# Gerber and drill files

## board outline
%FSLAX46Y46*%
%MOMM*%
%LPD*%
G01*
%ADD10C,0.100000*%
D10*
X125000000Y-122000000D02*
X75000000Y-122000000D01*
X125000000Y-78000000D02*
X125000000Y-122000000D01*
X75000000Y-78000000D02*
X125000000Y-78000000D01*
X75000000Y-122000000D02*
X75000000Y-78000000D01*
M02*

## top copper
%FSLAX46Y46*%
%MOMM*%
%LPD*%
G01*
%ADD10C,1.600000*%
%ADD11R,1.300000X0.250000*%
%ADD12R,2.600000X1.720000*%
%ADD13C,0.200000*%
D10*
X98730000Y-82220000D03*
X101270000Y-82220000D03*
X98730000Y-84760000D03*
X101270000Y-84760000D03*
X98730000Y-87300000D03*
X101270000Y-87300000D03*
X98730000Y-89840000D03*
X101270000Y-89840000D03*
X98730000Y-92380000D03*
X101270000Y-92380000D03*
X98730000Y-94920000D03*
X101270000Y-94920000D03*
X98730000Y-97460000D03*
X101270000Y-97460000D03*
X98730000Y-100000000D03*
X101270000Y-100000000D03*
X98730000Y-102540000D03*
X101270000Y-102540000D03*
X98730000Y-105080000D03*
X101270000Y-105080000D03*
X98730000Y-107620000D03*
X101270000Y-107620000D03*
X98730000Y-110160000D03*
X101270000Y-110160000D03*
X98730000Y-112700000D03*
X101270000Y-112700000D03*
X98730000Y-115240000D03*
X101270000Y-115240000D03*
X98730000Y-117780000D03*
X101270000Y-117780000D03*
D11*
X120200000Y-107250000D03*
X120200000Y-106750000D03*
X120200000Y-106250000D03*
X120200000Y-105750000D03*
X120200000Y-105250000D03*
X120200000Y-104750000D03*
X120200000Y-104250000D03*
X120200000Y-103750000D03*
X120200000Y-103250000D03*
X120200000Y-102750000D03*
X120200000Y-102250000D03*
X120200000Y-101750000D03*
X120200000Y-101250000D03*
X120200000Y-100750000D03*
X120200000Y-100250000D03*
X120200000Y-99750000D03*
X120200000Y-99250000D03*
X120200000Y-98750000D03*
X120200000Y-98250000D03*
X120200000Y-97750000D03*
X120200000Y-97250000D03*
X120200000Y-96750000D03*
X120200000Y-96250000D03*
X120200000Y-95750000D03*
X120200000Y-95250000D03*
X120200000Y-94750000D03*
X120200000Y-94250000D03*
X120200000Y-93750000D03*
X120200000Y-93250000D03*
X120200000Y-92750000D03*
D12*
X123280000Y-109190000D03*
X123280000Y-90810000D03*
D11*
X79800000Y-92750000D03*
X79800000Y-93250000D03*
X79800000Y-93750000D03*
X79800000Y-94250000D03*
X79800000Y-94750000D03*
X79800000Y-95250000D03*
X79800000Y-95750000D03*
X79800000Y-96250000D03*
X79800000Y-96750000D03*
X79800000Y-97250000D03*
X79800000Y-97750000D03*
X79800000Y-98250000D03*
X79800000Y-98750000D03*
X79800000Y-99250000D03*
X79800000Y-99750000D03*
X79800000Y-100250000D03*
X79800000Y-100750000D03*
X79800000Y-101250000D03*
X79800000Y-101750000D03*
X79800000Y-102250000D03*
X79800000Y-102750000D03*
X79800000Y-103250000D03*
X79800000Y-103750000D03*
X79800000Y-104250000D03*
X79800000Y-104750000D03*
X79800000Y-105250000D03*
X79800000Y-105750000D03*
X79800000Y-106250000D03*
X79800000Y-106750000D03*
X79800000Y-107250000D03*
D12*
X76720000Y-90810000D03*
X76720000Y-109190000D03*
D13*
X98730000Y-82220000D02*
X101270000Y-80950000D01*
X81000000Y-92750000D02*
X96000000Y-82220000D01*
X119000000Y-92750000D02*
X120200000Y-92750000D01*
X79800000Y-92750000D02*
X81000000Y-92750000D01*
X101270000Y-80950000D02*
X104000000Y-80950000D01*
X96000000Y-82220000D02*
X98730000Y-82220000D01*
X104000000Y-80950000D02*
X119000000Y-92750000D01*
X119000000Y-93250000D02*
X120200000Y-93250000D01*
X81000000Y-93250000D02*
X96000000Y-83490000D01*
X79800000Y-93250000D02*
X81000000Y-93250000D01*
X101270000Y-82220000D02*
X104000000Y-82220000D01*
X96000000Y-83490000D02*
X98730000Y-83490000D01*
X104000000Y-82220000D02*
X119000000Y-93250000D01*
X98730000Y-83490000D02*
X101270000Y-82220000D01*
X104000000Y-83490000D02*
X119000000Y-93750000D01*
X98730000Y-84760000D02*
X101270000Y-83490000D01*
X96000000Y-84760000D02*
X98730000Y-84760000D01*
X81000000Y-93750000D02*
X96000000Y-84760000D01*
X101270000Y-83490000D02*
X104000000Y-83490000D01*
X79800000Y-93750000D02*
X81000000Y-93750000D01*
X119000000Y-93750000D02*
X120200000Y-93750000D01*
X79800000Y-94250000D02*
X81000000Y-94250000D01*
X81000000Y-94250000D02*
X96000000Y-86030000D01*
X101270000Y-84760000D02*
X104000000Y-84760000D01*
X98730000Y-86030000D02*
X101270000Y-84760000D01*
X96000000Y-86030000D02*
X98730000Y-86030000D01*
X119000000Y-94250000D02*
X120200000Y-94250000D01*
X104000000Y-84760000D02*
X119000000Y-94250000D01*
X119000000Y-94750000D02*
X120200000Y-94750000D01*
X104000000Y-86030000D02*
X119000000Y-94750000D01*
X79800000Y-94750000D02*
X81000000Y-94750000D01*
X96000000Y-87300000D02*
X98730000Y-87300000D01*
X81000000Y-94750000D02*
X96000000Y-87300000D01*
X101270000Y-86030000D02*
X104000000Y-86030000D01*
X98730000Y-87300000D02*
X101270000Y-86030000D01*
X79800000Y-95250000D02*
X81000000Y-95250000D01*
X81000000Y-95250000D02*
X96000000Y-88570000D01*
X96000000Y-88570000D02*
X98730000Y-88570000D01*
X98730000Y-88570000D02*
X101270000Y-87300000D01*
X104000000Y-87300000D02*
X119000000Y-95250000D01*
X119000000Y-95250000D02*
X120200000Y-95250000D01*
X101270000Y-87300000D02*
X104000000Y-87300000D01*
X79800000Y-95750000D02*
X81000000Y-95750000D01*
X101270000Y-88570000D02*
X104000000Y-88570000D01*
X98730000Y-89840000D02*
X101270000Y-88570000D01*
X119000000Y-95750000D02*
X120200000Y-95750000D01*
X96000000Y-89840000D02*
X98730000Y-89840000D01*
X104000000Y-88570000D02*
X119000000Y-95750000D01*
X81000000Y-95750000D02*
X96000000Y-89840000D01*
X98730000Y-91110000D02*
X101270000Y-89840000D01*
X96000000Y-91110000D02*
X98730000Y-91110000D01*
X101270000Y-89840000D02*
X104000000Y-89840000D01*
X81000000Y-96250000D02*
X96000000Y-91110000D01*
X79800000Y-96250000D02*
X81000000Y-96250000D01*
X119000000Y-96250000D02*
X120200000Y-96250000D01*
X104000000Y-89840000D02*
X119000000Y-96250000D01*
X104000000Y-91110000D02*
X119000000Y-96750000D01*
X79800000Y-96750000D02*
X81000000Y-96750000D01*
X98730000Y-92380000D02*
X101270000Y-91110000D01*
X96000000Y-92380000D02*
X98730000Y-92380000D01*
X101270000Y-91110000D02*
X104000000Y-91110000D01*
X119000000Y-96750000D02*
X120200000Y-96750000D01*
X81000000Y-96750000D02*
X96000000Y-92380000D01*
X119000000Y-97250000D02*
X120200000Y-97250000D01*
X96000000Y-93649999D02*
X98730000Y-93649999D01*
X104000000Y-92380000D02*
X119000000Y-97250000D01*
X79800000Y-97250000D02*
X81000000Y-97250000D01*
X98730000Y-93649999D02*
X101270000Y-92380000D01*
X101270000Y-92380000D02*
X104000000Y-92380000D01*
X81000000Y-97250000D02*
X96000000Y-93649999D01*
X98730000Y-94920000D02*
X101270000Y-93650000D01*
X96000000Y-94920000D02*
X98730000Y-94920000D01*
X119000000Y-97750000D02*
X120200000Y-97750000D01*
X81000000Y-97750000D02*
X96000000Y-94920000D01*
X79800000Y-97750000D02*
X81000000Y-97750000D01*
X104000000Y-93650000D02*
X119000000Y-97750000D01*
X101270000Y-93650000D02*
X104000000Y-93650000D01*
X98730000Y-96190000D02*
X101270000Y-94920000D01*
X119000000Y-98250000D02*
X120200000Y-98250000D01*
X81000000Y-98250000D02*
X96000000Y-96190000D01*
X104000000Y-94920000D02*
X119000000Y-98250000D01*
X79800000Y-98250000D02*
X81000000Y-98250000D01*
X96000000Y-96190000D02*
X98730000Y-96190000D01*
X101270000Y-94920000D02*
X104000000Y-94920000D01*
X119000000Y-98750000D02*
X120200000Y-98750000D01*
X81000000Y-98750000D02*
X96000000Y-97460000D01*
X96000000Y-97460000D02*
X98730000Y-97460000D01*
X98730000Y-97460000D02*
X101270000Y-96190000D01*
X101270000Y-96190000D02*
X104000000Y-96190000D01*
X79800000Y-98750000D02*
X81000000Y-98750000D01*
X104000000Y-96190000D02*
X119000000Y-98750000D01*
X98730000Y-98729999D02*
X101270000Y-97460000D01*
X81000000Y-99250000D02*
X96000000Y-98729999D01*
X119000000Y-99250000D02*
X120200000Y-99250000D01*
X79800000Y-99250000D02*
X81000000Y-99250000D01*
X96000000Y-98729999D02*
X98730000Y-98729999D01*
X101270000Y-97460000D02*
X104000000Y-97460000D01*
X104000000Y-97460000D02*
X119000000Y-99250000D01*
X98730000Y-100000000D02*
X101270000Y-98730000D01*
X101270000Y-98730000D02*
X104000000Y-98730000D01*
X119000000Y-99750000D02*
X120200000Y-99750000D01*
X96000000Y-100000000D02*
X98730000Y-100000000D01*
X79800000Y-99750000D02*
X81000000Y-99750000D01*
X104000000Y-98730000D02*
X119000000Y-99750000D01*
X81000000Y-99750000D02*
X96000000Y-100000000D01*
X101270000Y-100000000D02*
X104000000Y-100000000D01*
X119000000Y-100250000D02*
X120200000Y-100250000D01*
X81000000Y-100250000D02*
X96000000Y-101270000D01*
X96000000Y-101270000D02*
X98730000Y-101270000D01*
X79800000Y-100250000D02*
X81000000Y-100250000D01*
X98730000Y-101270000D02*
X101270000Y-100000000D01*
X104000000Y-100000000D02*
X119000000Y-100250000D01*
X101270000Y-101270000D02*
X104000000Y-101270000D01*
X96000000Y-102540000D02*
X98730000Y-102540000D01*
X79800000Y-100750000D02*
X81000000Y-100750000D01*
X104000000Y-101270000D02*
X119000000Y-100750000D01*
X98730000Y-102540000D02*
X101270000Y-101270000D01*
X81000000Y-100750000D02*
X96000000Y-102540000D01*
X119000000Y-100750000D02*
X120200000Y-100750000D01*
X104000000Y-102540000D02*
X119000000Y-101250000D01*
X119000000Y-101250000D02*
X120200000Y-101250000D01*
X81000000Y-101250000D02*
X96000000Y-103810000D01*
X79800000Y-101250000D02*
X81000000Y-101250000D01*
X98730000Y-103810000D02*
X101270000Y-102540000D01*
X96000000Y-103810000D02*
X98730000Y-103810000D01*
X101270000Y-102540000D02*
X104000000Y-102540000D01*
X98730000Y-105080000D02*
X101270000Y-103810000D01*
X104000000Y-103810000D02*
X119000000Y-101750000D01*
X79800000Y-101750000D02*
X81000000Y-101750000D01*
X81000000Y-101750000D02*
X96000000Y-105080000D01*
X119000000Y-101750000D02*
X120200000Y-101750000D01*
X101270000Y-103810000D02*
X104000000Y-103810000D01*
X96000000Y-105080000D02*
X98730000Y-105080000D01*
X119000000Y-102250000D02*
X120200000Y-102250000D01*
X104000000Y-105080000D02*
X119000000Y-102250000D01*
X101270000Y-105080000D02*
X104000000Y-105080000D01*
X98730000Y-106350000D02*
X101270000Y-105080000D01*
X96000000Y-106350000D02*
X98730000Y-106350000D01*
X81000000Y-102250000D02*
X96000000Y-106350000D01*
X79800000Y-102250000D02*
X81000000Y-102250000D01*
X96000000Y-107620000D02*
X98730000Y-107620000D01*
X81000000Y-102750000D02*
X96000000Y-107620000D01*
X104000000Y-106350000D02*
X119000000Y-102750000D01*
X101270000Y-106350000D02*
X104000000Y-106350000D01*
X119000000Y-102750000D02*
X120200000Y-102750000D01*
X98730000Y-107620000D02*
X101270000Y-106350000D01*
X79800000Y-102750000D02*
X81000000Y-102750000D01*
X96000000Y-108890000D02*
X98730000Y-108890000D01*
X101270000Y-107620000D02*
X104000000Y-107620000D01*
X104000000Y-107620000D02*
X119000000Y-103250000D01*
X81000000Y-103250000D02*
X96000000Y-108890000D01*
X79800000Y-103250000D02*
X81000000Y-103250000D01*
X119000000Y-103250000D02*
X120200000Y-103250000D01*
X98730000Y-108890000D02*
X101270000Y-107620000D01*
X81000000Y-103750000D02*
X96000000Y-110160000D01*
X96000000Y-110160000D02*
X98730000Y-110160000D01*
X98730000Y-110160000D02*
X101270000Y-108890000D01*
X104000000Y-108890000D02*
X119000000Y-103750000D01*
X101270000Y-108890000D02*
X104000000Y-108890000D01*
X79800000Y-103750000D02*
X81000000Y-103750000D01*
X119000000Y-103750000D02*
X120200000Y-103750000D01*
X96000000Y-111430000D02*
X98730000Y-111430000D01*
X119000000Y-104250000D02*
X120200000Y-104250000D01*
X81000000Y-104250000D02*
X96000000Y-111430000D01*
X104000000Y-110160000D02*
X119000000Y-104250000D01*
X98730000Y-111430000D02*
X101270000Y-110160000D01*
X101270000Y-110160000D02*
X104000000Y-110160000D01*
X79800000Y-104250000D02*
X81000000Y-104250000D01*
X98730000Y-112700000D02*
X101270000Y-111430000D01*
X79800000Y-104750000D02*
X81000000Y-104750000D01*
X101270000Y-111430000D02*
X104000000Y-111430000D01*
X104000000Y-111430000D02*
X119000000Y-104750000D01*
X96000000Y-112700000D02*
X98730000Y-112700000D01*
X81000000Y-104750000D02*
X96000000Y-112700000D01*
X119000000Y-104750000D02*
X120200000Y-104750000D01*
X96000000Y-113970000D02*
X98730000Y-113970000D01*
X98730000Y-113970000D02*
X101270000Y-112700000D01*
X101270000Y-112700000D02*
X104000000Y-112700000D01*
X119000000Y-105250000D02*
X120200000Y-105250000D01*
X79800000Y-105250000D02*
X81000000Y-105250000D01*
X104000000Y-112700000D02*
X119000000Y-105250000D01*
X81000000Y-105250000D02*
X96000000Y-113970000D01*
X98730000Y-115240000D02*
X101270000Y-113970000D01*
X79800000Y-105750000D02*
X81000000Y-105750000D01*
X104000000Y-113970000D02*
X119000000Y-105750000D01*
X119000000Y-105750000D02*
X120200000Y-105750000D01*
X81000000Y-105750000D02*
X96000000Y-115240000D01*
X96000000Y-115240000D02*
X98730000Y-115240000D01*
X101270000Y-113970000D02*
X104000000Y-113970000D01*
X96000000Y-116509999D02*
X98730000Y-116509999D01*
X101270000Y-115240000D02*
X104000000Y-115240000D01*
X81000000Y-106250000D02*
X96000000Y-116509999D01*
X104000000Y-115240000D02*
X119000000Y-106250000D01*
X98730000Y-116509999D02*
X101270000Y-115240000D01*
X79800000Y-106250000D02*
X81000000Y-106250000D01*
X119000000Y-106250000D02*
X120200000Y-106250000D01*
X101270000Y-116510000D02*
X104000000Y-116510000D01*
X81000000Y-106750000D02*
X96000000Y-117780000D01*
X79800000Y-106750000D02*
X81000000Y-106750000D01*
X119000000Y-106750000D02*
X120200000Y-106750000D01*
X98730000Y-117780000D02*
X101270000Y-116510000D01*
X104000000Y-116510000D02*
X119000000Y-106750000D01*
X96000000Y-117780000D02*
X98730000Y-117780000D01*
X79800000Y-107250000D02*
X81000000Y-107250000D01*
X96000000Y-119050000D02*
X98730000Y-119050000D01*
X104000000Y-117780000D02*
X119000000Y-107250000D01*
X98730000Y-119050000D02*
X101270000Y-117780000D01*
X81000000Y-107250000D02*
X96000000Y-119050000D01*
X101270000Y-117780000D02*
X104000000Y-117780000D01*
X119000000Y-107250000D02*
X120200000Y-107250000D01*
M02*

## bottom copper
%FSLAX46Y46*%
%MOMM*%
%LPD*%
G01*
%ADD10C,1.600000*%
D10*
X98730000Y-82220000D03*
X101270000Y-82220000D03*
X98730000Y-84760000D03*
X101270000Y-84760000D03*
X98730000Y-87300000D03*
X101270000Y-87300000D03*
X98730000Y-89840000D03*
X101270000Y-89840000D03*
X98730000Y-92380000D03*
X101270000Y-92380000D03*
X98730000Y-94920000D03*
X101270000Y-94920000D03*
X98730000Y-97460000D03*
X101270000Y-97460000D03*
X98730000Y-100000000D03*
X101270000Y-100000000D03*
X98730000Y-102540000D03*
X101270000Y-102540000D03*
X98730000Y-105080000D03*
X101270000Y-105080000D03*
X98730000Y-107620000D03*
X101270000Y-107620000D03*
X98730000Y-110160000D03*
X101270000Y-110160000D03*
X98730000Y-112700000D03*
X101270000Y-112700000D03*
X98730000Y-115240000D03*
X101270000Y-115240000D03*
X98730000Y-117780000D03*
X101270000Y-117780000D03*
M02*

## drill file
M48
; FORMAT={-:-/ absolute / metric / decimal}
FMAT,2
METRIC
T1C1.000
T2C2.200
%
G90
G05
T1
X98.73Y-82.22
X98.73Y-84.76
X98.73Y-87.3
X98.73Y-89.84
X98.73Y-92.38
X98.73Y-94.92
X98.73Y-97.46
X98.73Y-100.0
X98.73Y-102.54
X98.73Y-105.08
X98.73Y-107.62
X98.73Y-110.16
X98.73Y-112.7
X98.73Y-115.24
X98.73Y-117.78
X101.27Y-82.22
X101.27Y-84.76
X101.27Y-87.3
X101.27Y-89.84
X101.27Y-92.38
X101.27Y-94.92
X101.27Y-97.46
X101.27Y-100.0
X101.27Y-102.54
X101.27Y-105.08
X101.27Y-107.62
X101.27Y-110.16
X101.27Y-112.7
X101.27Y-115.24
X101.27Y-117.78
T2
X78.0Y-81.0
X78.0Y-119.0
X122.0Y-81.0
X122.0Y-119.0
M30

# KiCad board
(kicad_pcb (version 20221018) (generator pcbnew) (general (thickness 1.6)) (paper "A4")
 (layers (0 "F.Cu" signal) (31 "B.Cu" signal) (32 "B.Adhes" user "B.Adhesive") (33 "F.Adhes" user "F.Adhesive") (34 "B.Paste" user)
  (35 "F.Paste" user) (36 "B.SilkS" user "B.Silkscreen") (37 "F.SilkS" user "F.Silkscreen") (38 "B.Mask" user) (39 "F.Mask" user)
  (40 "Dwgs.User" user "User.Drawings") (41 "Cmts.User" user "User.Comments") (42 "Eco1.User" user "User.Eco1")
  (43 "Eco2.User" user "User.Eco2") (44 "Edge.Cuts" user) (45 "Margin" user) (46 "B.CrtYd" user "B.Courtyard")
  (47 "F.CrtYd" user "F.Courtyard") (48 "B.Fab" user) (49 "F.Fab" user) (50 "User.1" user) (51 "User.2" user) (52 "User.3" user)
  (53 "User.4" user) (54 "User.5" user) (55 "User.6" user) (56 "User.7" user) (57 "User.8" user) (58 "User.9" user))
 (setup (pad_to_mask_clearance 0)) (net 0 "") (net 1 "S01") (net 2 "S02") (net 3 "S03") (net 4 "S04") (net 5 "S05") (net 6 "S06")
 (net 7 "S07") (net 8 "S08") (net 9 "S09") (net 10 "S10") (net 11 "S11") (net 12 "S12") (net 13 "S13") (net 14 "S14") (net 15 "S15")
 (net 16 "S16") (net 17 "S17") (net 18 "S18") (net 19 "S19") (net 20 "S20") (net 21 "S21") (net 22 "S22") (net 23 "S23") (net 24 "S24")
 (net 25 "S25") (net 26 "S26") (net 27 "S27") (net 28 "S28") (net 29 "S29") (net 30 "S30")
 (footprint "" (layer "F.Cu") (at 122 119)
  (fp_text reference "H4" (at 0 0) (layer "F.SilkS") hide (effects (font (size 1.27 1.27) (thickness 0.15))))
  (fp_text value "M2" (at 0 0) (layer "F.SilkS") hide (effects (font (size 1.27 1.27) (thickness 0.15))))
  (pad "" np_thru_hole circle (at 0 0) (size 2.2 2.2) (drill 2.2) (layers "F&B.Cu" "*.Mask")))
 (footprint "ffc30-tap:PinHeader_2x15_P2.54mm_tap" (layer "F.Cu") (at 100 100)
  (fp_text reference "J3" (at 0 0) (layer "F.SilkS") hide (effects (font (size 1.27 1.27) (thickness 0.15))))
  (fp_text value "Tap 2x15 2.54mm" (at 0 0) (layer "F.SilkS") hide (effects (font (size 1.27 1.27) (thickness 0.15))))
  (pad "1" thru_hole circle (at -1.27 -17.78) (size 1.6 1.6) (drill 1) (layers "*.Cu" "*.Mask") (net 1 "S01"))
  (pad "2" thru_hole circle (at 1.27 -17.78) (size 1.6 1.6) (drill 1) (layers "*.Cu" "*.Mask") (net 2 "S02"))
  (pad "3" thru_hole circle (at -1.27 -15.24) (size 1.6 1.6) (drill 1) (layers "*.Cu" "*.Mask") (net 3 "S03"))
  (pad "4" thru_hole circle (at 1.27 -15.24) (size 1.6 1.6) (drill 1) (layers "*.Cu" "*.Mask") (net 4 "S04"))
  (pad "5" thru_hole circle (at -1.27 -12.7) (size 1.6 1.6) (drill 1) (layers "*.Cu" "*.Mask") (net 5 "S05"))
  (pad "6" thru_hole circle (at 1.27 -12.7) (size 1.6 1.6) (drill 1) (layers "*.Cu" "*.Mask") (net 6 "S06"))
  (pad "7" thru_hole circle (at -1.27 -10.16) (size 1.6 1.6) (drill 1) (layers "*.Cu" "*.Mask") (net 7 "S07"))
  (pad "8" thru_hole circle (at 1.27 -10.16) (size 1.6 1.6) (drill 1) (layers "*.Cu" "*.Mask") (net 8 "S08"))
  (pad "9" thru_hole circle (at -1.27 -7.62) (size 1.6 1.6) (drill 1) (layers "*.Cu" "*.Mask") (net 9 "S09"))
  (pad "10" thru_hole circle (at 1.27 -7.62) (size 1.6 1.6) (drill 1) (layers "*.Cu" "*.Mask") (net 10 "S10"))
  (pad "11" thru_hole circle (at -1.27 -5.08) (size 1.6 1.6) (drill 1) (layers "*.Cu" "*.Mask") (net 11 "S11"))
  (pad "12" thru_hole circle (at 1.27 -5.08) (size 1.6 1.6) (drill 1) (layers "*.Cu" "*.Mask") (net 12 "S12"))
  (pad "13" thru_hole circle (at -1.27 -2.54) (size 1.6 1.6) (drill 1) (layers "*.Cu" "*.Mask") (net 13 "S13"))
  (pad "14" thru_hole circle (at 1.27 -2.54) (size 1.6 1.6) (drill 1) (layers "*.Cu" "*.Mask") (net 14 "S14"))
  (pad "15" thru_hole circle (at -1.27 0) (size 1.6 1.6) (drill 1) (layers "*.Cu" "*.Mask") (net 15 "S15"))
  (pad "16" thru_hole circle (at 1.27 0) (size 1.6 1.6) (drill 1) (layers "*.Cu" "*.Mask") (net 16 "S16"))
  (pad "17" thru_hole circle (at -1.27 2.54) (size 1.6 1.6) (drill 1) (layers "*.Cu" "*.Mask") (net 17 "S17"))
  (pad "18" thru_hole circle (at 1.27 2.54) (size 1.6 1.6) (drill 1) (layers "*.Cu" "*.Mask") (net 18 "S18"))
  (pad "19" thru_hole circle (at -1.27 5.08) (size 1.6 1.6) (drill 1) (layers "*.Cu" "*.Mask") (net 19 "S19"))
  (pad "20" thru_hole circle (at 1.27 5.08) (size 1.6 1.6) (drill 1) (layers "*.Cu" "*.Mask") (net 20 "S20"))
  (pad "21" thru_hole circle (at -1.27 7.62) (size 1.6 1.6) (drill 1) (layers "*.Cu" "*.Mask") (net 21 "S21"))
  (pad "22" thru_hole circle (at 1.27 7.62) (size 1.6 1.6) (drill 1) (layers "*.Cu" "*.Mask") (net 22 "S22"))
  (pad "23" thru_hole circle (at -1.27 10.16) (size 1.6 1.6) (drill 1) (layers "*.Cu" "*.Mask") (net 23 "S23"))
  (pad "24" thru_hole circle (at 1.27 10.16) (size 1.6 1.6) (drill 1) (layers "*.Cu" "*.Mask") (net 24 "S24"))
  (pad "25" thru_hole circle (at -1.27 12.7) (size 1.6 1.6) (drill 1) (layers "*.Cu" "*.Mask") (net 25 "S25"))
  (pad "26" thru_hole circle (at 1.27 12.7) (size 1.6 1.6) (drill 1) (layers "*.Cu" "*.Mask") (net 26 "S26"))
  (pad "27" thru_hole circle (at -1.27 15.24) (size 1.6 1.6) (drill 1) (layers "*.Cu" "*.Mask") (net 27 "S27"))
  (pad "28" thru_hole circle (at 1.27 15.24) (size 1.6 1.6) (drill 1) (layers "*.Cu" "*.Mask") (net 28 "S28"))
  (pad "29" thru_hole circle (at -1.27 17.78) (size 1.6 1.6) (drill 1) (layers "*.Cu" "*.Mask") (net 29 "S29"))
  (pad "30" thru_hole circle (at 1.27 17.78) (size 1.6 1.6) (drill 1) (layers "*.Cu" "*.Mask") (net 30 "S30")))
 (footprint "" (layer "F.Cu") (at 122 81)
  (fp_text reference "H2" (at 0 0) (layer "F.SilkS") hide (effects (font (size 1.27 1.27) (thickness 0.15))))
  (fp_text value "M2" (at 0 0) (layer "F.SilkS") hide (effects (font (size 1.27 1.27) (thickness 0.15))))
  (pad "" np_thru_hole circle (at 0 0) (size 2.2 2.2) (drill 2.2) (layers "F&B.Cu" "*.Mask")))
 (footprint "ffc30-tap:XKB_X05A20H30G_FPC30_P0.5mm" (layer "F.Cu") (at 122.065 100 90)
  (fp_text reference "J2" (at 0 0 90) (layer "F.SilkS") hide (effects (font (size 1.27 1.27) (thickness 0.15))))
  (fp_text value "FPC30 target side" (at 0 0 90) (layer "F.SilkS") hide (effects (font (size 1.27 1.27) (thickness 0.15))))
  (pad "1" smd rect (at -7.25 -1.865 90) (size 0.25 1.3) (layers "F.Cu" "F.Paste" "F.Mask") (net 30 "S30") (thermal_bridge_angle 45))
  (pad "2" smd rect (at -6.75 -1.865 90) (size 0.25 1.3) (layers "F.Cu" "F.Paste" "F.Mask") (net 29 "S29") (thermal_bridge_angle 45))
  (pad "3" smd rect (at -6.25 -1.865 90) (size 0.25 1.3) (layers "F.Cu" "F.Paste" "F.Mask") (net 28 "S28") (thermal_bridge_angle 45))
  (pad "4" smd rect (at -5.75 -1.865 90) (size 0.25 1.3) (layers "F.Cu" "F.Paste" "F.Mask") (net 27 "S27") (thermal_bridge_angle 45))
  (pad "5" smd rect (at -5.25 -1.865 90) (size 0.25 1.3) (layers "F.Cu" "F.Paste" "F.Mask") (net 26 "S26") (thermal_bridge_angle 45))
  (pad "6" smd rect (at -4.75 -1.865 90) (size 0.25 1.3) (layers "F.Cu" "F.Paste" "F.Mask") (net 25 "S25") (thermal_bridge_angle 45))
  (pad "7" smd rect (at -4.25 -1.865 90) (size 0.25 1.3) (layers "F.Cu" "F.Paste" "F.Mask") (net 24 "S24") (thermal_bridge_angle 45))
  (pad "8" smd rect (at -3.75 -1.865 90) (size 0.25 1.3) (layers "F.Cu" "F.Paste" "F.Mask") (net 23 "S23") (thermal_bridge_angle 45))
  (pad "9" smd rect (at -3.25 -1.865 90) (size 0.25 1.3) (layers "F.Cu" "F.Paste" "F.Mask") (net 22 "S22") (thermal_bridge_angle 45))
  (pad "10" smd rect (at -2.75 -1.865 90) (size 0.25 1.3) (layers "F.Cu" "F.Paste" "F.Mask") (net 21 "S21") (thermal_bridge_angle 45))
  (pad "11" smd rect (at -2.25 -1.865 90) (size 0.25 1.3) (layers "F.Cu" "F.Paste" "F.Mask") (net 20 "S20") (thermal_bridge_angle 45))
  (pad "12" smd rect (at -1.75 -1.865 90) (size 0.25 1.3) (layers "F.Cu" "F.Paste" "F.Mask") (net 19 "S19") (thermal_bridge_angle 45))
  (pad "13" smd rect (at -1.25 -1.865 90) (size 0.25 1.3) (layers "F.Cu" "F.Paste" "F.Mask") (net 18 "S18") (thermal_bridge_angle 45))
  (pad "14" smd rect (at -0.75 -1.865 90) (size 0.25 1.3) (layers "F.Cu" "F.Paste" "F.Mask") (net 17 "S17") (thermal_bridge_angle 45))
  (pad "15" smd rect (at -0.25 -1.865 90) (size 0.25 1.3) (layers "F.Cu" "F.Paste" "F.Mask") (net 16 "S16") (thermal_bridge_angle 45))
  (pad "16" smd rect (at 0.25 -1.865 90) (size 0.25 1.3) (layers "F.Cu" "F.Paste" "F.Mask") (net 15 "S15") (thermal_bridge_angle 45))
  (pad "17" smd rect (at 0.75 -1.865 90) (size 0.25 1.3) (layers "F.Cu" "F.Paste" "F.Mask") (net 14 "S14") (thermal_bridge_angle 45))
  (pad "18" smd rect (at 1.25 -1.865 90) (size 0.25 1.3) (layers "F.Cu" "F.Paste" "F.Mask") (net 13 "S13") (thermal_bridge_angle 45))
  (pad "19" smd rect (at 1.75 -1.865 90) (size 0.25 1.3) (layers "F.Cu" "F.Paste" "F.Mask") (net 12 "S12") (thermal_bridge_angle 45))
  (pad "20" smd rect (at 2.25 -1.865 90) (size 0.25 1.3) (layers "F.Cu" "F.Paste" "F.Mask") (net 11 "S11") (thermal_bridge_angle 45))
  (pad "21" smd rect (at 2.75 -1.865 90) (size 0.25 1.3) (layers "F.Cu" "F.Paste" "F.Mask") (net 10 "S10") (thermal_bridge_angle 45))
  (pad "22" smd rect (at 3.25 -1.865 90) (size 0.25 1.3) (layers "F.Cu" "F.Paste" "F.Mask") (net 9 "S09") (thermal_bridge_angle 45))
  (pad "23" smd rect (at 3.75 -1.865 90) (size 0.25 1.3) (layers "F.Cu" "F.Paste" "F.Mask") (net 8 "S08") (thermal_bridge_angle 45))
  (pad "24" smd rect (at 4.25 -1.865 90) (size 0.25 1.3) (layers "F.Cu" "F.Paste" "F.Mask") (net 7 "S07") (thermal_bridge_angle 45))
  (pad "25" smd rect (at 4.75 -1.865 90) (size 0.25 1.3) (layers "F.Cu" "F.Paste" "F.Mask") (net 6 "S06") (thermal_bridge_angle 45))
  (pad "26" smd rect (at 5.25 -1.865 90) (size 0.25 1.3) (layers "F.Cu" "F.Paste" "F.Mask") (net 5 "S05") (thermal_bridge_angle 45))
  (pad "27" smd rect (at 5.75 -1.865 90) (size 0.25 1.3) (layers "F.Cu" "F.Paste" "F.Mask") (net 4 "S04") (thermal_bridge_angle 45))
  (pad "28" smd rect (at 6.25 -1.865 90) (size 0.25 1.3) (layers "F.Cu" "F.Paste" "F.Mask") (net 3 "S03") (thermal_bridge_angle 45))
  (pad "29" smd rect (at 6.75 -1.865 90) (size 0.25 1.3) (layers "F.Cu" "F.Paste" "F.Mask") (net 2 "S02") (thermal_bridge_angle 45))
  (pad "30" smd rect (at 7.25 -1.865 90) (size 0.25 1.3) (layers "F.Cu" "F.Paste" "F.Mask") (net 1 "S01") (thermal_bridge_angle 45))
  (pad "MP" smd rect (at -9.19 1.215 90) (size 1.72 2.6) (layers "F.Cu" "F.Paste" "F.Mask") (thermal_bridge_angle 45))
  (pad "MP" smd rect (at 9.19 1.215 90) (size 1.72 2.6) (layers "F.Cu" "F.Paste" "F.Mask") (thermal_bridge_angle 45)))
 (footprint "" (layer "F.Cu") (at 78 119)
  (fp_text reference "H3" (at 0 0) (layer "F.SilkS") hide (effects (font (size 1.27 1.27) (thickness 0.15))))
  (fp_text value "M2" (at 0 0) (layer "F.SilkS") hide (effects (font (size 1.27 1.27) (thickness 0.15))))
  (pad "" np_thru_hole circle (at 0 0) (size 2.2 2.2) (drill 2.2) (layers "F&B.Cu" "*.Mask")))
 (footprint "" (layer "F.Cu") (at 78 81)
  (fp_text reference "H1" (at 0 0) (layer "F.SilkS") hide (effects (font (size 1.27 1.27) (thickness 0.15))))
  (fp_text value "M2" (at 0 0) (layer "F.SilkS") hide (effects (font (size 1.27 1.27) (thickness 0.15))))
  (pad "" np_thru_hole circle (at 0 0) (size 2.2 2.2) (drill 2.2) (layers "F&B.Cu" "*.Mask")))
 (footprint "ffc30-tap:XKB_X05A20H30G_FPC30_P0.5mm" (layer "F.Cu") (at 77.935 100 -90)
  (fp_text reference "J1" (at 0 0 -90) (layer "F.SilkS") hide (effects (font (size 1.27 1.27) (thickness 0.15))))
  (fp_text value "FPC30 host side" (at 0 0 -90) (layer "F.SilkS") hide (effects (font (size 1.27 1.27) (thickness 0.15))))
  (pad "1" smd rect (at -7.25 -1.865 270) (size 0.25 1.3) (layers "F.Cu" "F.Paste" "F.Mask") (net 1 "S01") (thermal_bridge_angle 45))
  (pad "2" smd rect (at -6.75 -1.865 270) (size 0.25 1.3) (layers "F.Cu" "F.Paste" "F.Mask") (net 2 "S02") (thermal_bridge_angle 45))
  (pad "3" smd rect (at -6.25 -1.865 270) (size 0.25 1.3) (layers "F.Cu" "F.Paste" "F.Mask") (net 3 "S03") (thermal_bridge_angle 45))
  (pad "4" smd rect (at -5.75 -1.865 270) (size 0.25 1.3) (layers "F.Cu" "F.Paste" "F.Mask") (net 4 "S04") (thermal_bridge_angle 45))
  (pad "5" smd rect (at -5.25 -1.865 270) (size 0.25 1.3) (layers "F.Cu" "F.Paste" "F.Mask") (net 5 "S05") (thermal_bridge_angle 45))
  (pad "6" smd rect (at -4.75 -1.865 270) (size 0.25 1.3) (layers "F.Cu" "F.Paste" "F.Mask") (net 6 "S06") (thermal_bridge_angle 45))
  (pad "7" smd rect (at -4.25 -1.865 270) (size 0.25 1.3) (layers "F.Cu" "F.Paste" "F.Mask") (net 7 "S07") (thermal_bridge_angle 45))
  (pad "8" smd rect (at -3.75 -1.865 270) (size 0.25 1.3) (layers "F.Cu" "F.Paste" "F.Mask") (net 8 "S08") (thermal_bridge_angle 45))
  (pad "9" smd rect (at -3.25 -1.865 270) (size 0.25 1.3) (layers "F.Cu" "F.Paste" "F.Mask") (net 9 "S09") (thermal_bridge_angle 45))
  (pad "10" smd rect (at -2.75 -1.865 270) (size 0.25 1.3) (layers "F.Cu" "F.Paste" "F.Mask") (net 10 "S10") (thermal_bridge_angle 45))
  (pad "11" smd rect (at -2.25 -1.865 270) (size 0.25 1.3) (layers "F.Cu" "F.Paste" "F.Mask") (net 11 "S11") (thermal_bridge_angle 45))
  (pad "12" smd rect (at -1.75 -1.865 270) (size 0.25 1.3) (layers "F.Cu" "F.Paste" "F.Mask") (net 12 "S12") (thermal_bridge_angle 45))
  (pad "13" smd rect (at -1.25 -1.865 270) (size 0.25 1.3) (layers "F.Cu" "F.Paste" "F.Mask") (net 13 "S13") (thermal_bridge_angle 45))
  (pad "14" smd rect (at -0.75 -1.865 270) (size 0.25 1.3) (layers "F.Cu" "F.Paste" "F.Mask") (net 14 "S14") (thermal_bridge_angle 45))
  (pad "15" smd rect (at -0.25 -1.865 270) (size 0.25 1.3) (layers "F.Cu" "F.Paste" "F.Mask") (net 15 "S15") (thermal_bridge_angle 45))
  (pad "16" smd rect (at 0.25 -1.865 270) (size 0.25 1.3) (layers "F.Cu" "F.Paste" "F.Mask") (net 16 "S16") (thermal_bridge_angle 45))
  (pad "17" smd rect (at 0.75 -1.865 270) (size 0.25 1.3) (layers "F.Cu" "F.Paste" "F.Mask") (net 17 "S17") (thermal_bridge_angle 45))
  (pad "18" smd rect (at 1.25 -1.865 270) (size 0.25 1.3) (layers "F.Cu" "F.Paste" "F.Mask") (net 18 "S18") (thermal_bridge_angle 45))
  (pad "19" smd rect (at 1.75 -1.865 270) (size 0.25 1.3) (layers "F.Cu" "F.Paste" "F.Mask") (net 19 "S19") (thermal_bridge_angle 45))
  (pad "20" smd rect (at 2.25 -1.865 270) (size 0.25 1.3) (layers "F.Cu" "F.Paste" "F.Mask") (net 20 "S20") (thermal_bridge_angle 45))
  (pad "21" smd rect (at 2.75 -1.865 270) (size 0.25 1.3) (layers "F.Cu" "F.Paste" "F.Mask") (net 21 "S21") (thermal_bridge_angle 45))
  (pad "22" smd rect (at 3.25 -1.865 270) (size 0.25 1.3) (layers "F.Cu" "F.Paste" "F.Mask") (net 22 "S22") (thermal_bridge_angle 45))
  (pad "23" smd rect (at 3.75 -1.865 270) (size 0.25 1.3) (layers "F.Cu" "F.Paste" "F.Mask") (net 23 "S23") (thermal_bridge_angle 45))
  (pad "24" smd rect (at 4.25 -1.865 270) (size 0.25 1.3) (layers "F.Cu" "F.Paste" "F.Mask") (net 24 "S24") (thermal_bridge_angle 45))
  (pad "25" smd rect (at 4.75 -1.865 270) (size 0.25 1.3) (layers "F.Cu" "F.Paste" "F.Mask") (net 25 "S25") (thermal_bridge_angle 45))
  (pad "26" smd rect (at 5.25 -1.865 270) (size 0.25 1.3) (layers "F.Cu" "F.Paste" "F.Mask") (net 26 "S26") (thermal_bridge_angle 45))
  (pad "27" smd rect (at 5.75 -1.865 270) (size 0.25 1.3) (layers "F.Cu" "F.Paste" "F.Mask") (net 27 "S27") (thermal_bridge_angle 45))
  (pad "28" smd rect (at 6.25 -1.865 270) (size 0.25 1.3) (layers "F.Cu" "F.Paste" "F.Mask") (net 28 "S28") (thermal_bridge_angle 45))
  (pad "29" smd rect (at 6.75 -1.865 270) (size 0.25 1.3) (layers "F.Cu" "F.Paste" "F.Mask") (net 29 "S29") (thermal_bridge_angle 45))
  (pad "30" smd rect (at 7.25 -1.865 270) (size 0.25 1.3) (layers "F.Cu" "F.Paste" "F.Mask") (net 30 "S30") (thermal_bridge_angle 45))
  (pad "MP" smd rect (at -9.19 1.215 270) (size 1.72 2.6) (layers "F.Cu" "F.Paste" "F.Mask") (thermal_bridge_angle 45))
  (pad "MP" smd rect (at 9.19 1.215 270) (size 1.72 2.6) (layers "F.Cu" "F.Paste" "F.Mask") (thermal_bridge_angle 45)))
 (gr_line (start 125 122) (end 75 122) (stroke (width 0.1) (type default)) (layer "Edge.Cuts"))
 (gr_line (start 125 78) (end 125 122) (stroke (width 0.1) (type default)) (layer "Edge.Cuts"))
 (gr_line (start 75 78) (end 125 78) (stroke (width 0.1) (type default)) (layer "Edge.Cuts"))
 (gr_line (start 75 122) (end 75 78) (stroke (width 0.1) (type default)) (layer "Edge.Cuts"))
 (segment (start 98.73 82.22) (end 101.27 80.95) (width 0.2) (layer "F.Cu") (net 1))
 (segment (start 81 92.75) (end 96 82.22) (width 0.2) (layer "F.Cu") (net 1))
 (segment (start 119 92.75) (end 120.2 92.75) (width 0.2) (layer "F.Cu") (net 1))
 (segment (start 79.8 92.75) (end 81 92.75) (width 0.2) (layer "F.Cu") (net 1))
 (segment (start 101.27 80.95) (end 104 80.95) (width 0.2) (layer "F.Cu") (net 1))
 (segment (start 96 82.22) (end 98.73 82.22) (width 0.2) (layer "F.Cu") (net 1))
 (segment (start 104 80.95) (end 119 92.75) (width 0.2) (layer "F.Cu") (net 1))
 (segment (start 119 93.25) (end 120.2 93.25) (width 0.2) (layer "F.Cu") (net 2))
 (segment (start 81 93.25) (end 96 83.49) (width 0.2) (layer "F.Cu") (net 2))
 (segment (start 79.8 93.25) (end 81 93.25) (width 0.2) (layer "F.Cu") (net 2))
 (segment (start 101.27 82.22) (end 104 82.22) (width 0.2) (layer "F.Cu") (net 2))
 (segment (start 96 83.49) (end 98.73 83.49) (width 0.2) (layer "F.Cu") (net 2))
 (segment (start 104 82.22) (end 119 93.25) (width 0.2) (layer "F.Cu") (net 2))
 (segment (start 98.73 83.49) (end 101.27 82.22) (width 0.2) (layer "F.Cu") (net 2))
 (segment (start 104 83.49) (end 119 93.75) (width 0.2) (layer "F.Cu") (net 3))
 (segment (start 98.73 84.76) (end 101.27 83.49) (width 0.2) (layer "F.Cu") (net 3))
 (segment (start 96 84.76) (end 98.73 84.76) (width 0.2) (layer "F.Cu") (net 3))
 (segment (start 81 93.75) (end 96 84.76) (width 0.2) (layer "F.Cu") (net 3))
 (segment (start 101.27 83.49) (end 104 83.49) (width 0.2) (layer "F.Cu") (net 3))
 (segment (start 79.8 93.75) (end 81 93.75) (width 0.2) (layer "F.Cu") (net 3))
 (segment (start 119 93.75) (end 120.2 93.75) (width 0.2) (layer "F.Cu") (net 3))
 (segment (start 79.8 94.25) (end 81 94.25) (width 0.2) (layer "F.Cu") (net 4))
 (segment (start 81 94.25) (end 96 86.03) (width 0.2) (layer "F.Cu") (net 4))
 (segment (start 101.27 84.76) (end 104 84.76) (width 0.2) (layer "F.Cu") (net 4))
 (segment (start 98.73 86.03) (end 101.27 84.76) (width 0.2) (layer "F.Cu") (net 4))
 (segment (start 96 86.03) (end 98.73 86.03) (width 0.2) (layer "F.Cu") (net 4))
 (segment (start 119 94.25) (end 120.2 94.25) (width 0.2) (layer "F.Cu") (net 4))
 (segment (start 104 84.76) (end 119 94.25) (width 0.2) (layer "F.Cu") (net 4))
 (segment (start 119 94.75) (end 120.2 94.75) (width 0.2) (layer "F.Cu") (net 5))
 (segment (start 104 86.03) (end 119 94.75) (width 0.2) (layer "F.Cu") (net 5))
 (segment (start 79.8 94.75) (end 81 94.75) (width 0.2) (layer "F.Cu") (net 5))
 (segment (start 96 87.3) (end 98.73 87.3) (width 0.2) (layer "F.Cu") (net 5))
 (segment (start 81 94.75) (end 96 87.3) (width 0.2) (layer "F.Cu") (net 5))
 (segment (start 101.27 86.03) (end 104 86.03) (width 0.2) (layer "F.Cu") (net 5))
 (segment (start 98.73 87.3) (end 101.27 86.03) (width 0.2) (layer "F.Cu") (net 5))
 (segment (start 79.8 95.25) (end 81 95.25) (width 0.2) (layer "F.Cu") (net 6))
 (segment (start 81 95.25) (end 96 88.57) (width 0.2) (layer "F.Cu") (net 6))
 (segment (start 96 88.57) (end 98.73 88.57) (width 0.2) (layer "F.Cu") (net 6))
 (segment (start 98.73 88.57) (end 101.27 87.3) (width 0.2) (layer "F.Cu") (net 6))
 (segment (start 104 87.3) (end 119 95.25) (width 0.2) (layer "F.Cu") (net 6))
 (segment (start 119 95.25) (end 120.2 95.25) (width 0.2) (layer "F.Cu") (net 6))
 (segment (start 101.27 87.3) (end 104 87.3) (width 0.2) (layer "F.Cu") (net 6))
 (segment (start 79.8 95.75) (end 81 95.75) (width 0.2) (layer "F.Cu") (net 7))
 (segment (start 101.27 88.57) (end 104 88.57) (width 0.2) (layer "F.Cu") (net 7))
 (segment (start 98.73 89.84) (end 101.27 88.57) (width 0.2) (layer "F.Cu") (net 7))
 (segment (start 119 95.75) (end 120.2 95.75) (width 0.2) (layer "F.Cu") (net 7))
 (segment (start 96 89.84) (end 98.73 89.84) (width 0.2) (layer "F.Cu") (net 7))
 (segment (start 104 88.57) (end 119 95.75) (width 0.2) (layer "F.Cu") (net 7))
 (segment (start 81 95.75) (end 96 89.84) (width 0.2) (layer "F.Cu") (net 7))
 (segment (start 98.73 91.11) (end 101.27 89.84) (width 0.2) (layer "F.Cu") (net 8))
 (segment (start 96 91.11) (end 98.73 91.11) (width 0.2) (layer "F.Cu") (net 8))
 (segment (start 101.27 89.84) (end 104 89.84) (width 0.2) (layer "F.Cu") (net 8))
 (segment (start 81 96.25) (end 96 91.11) (width 0.2) (layer "F.Cu") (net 8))
 (segment (start 79.8 96.25) (end 81 96.25) (width 0.2) (layer "F.Cu") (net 8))
 (segment (start 119 96.25) (end 120.2 96.25) (width 0.2) (layer "F.Cu") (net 8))
 (segment (start 104 89.84) (end 119 96.25) (width 0.2) (layer "F.Cu") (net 8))
 (segment (start 104 91.11) (end 119 96.75) (width 0.2) (layer "F.Cu") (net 9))
 (segment (start 79.8 96.75) (end 81 96.75) (width 0.2) (layer "F.Cu") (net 9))
 (segment (start 98.73 92.38) (end 101.27 91.11) (width 0.2) (layer "F.Cu") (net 9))
 (segment (start 96 92.38) (end 98.73 92.38) (width 0.2) (layer "F.Cu") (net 9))
 (segment (start 101.27 91.11) (end 104 91.11) (width 0.2) (layer "F.Cu") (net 9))
 (segment (start 119 96.75) (end 120.2 96.75) (width 0.2) (layer "F.Cu") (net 9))
 (segment (start 81 96.75) (end 96 92.38) (width 0.2) (layer "F.Cu") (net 9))
 (segment (start 119 97.25) (end 120.2 97.25) (width 0.2) (layer "F.Cu") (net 10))
 (segment (start 96 93.649999) (end 98.73 93.649999) (width 0.2) (layer "F.Cu") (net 10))
 (segment (start 104 92.38) (end 119 97.25) (width 0.2) (layer "F.Cu") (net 10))
 (segment (start 79.8 97.25) (end 81 97.25) (width 0.2) (layer "F.Cu") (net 10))
 (segment (start 98.73 93.649999) (end 101.27 92.38) (width 0.2) (layer "F.Cu") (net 10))
 (segment (start 101.27 92.38) (end 104 92.38) (width 0.2) (layer "F.Cu") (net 10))
 (segment (start 81 97.25) (end 96 93.649999) (width 0.2) (layer "F.Cu") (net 10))
 (segment (start 98.73 94.92) (end 101.27 93.65) (width 0.2) (layer "F.Cu") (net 11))
 (segment (start 96 94.92) (end 98.73 94.92) (width 0.2) (layer "F.Cu") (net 11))
 (segment (start 119 97.75) (end 120.2 97.75) (width 0.2) (layer "F.Cu") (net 11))
 (segment (start 81 97.75) (end 96 94.92) (width 0.2) (layer "F.Cu") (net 11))
 (segment (start 79.8 97.75) (end 81 97.75) (width 0.2) (layer "F.Cu") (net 11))
 (segment (start 104 93.65) (end 119 97.75) (width 0.2) (layer "F.Cu") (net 11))
 (segment (start 101.27 93.65) (end 104 93.65) (width 0.2) (layer "F.Cu") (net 11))
 (segment (start 98.73 96.19) (end 101.27 94.92) (width 0.2) (layer "F.Cu") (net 12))
 (segment (start 119 98.25) (end 120.2 98.25) (width 0.2) (layer "F.Cu") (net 12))
 (segment (start 81 98.25) (end 96 96.19) (width 0.2) (layer "F.Cu") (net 12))
 (segment (start 104 94.92) (end 119 98.25) (width 0.2) (layer "F.Cu") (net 12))
 (segment (start 79.8 98.25) (end 81 98.25) (width 0.2) (layer "F.Cu") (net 12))
 (segment (start 96 96.19) (end 98.73 96.19) (width 0.2) (layer "F.Cu") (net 12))
 (segment (start 101.27 94.92) (end 104 94.92) (width 0.2) (layer "F.Cu") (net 12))
 (segment (start 119 98.75) (end 120.2 98.75) (width 0.2) (layer "F.Cu") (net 13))
 (segment (start 81 98.75) (end 96 97.46) (width 0.2) (layer "F.Cu") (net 13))
 (segment (start 96 97.46) (end 98.73 97.46) (width 0.2) (layer "F.Cu") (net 13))
 (segment (start 98.73 97.46) (end 101.27 96.19) (width 0.2) (layer "F.Cu") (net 13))
 (segment (start 101.27 96.19) (end 104 96.19) (width 0.2) (layer "F.Cu") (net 13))
 (segment (start 79.8 98.75) (end 81 98.75) (width 0.2) (layer "F.Cu") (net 13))
 (segment (start 104 96.19) (end 119 98.75) (width 0.2) (layer "F.Cu") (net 13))
 (segment (start 98.73 98.729999) (end 101.27 97.46) (width 0.2) (layer "F.Cu") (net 14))
 (segment (start 81 99.25) (end 96 98.729999) (width 0.2) (layer "F.Cu") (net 14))
 (segment (start 119 99.25) (end 120.2 99.25) (width 0.2) (layer "F.Cu") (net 14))
 (segment (start 79.8 99.25) (end 81 99.25) (width 0.2) (layer "F.Cu") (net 14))
 (segment (start 96 98.729999) (end 98.73 98.729999) (width 0.2) (layer "F.Cu") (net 14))
 (segment (start 101.27 97.46) (end 104 97.46) (width 0.2) (layer "F.Cu") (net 14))
 (segment (start 104 97.46) (end 119 99.25) (width 0.2) (layer "F.Cu") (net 14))
 (segment (start 98.73 100) (end 101.27 98.73) (width 0.2) (layer "F.Cu") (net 15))
 (segment (start 101.27 98.73) (end 104 98.73) (width 0.2) (layer "F.Cu") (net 15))
 (segment (start 119 99.75) (end 120.2 99.75) (width 0.2) (layer "F.Cu") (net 15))
 (segment (start 96 100) (end 98.73 100) (width 0.2) (layer "F.Cu") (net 15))
 (segment (start 79.8 99.75) (end 81 99.75) (width 0.2) (layer "F.Cu") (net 15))
 (segment (start 104 98.73) (end 119 99.75) (width 0.2) (layer "F.Cu") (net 15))
 (segment (start 81 99.75) (end 96 100) (width 0.2) (layer "F.Cu") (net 15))
 (segment (start 101.27 100) (end 104 100) (width 0.2) (layer "F.Cu") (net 16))
 (segment (start 119 100.25) (end 120.2 100.25) (width 0.2) (layer "F.Cu") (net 16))
 (segment (start 81 100.25) (end 96 101.27) (width 0.2) (layer "F.Cu") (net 16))
 (segment (start 96 101.27) (end 98.73 101.27) (width 0.2) (layer "F.Cu") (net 16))
 (segment (start 79.8 100.25) (end 81 100.25) (width 0.2) (layer "F.Cu") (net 16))
 (segment (start 98.73 101.27) (end 101.27 100) (width 0.2) (layer "F.Cu") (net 16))
 (segment (start 104 100) (end 119 100.25) (width 0.2) (layer "F.Cu") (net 16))
 (segment (start 101.27 101.27) (end 104 101.27) (width 0.2) (layer "F.Cu") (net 17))
 (segment (start 96 102.54) (end 98.73 102.54) (width 0.2) (layer "F.Cu") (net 17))
 (segment (start 79.8 100.75) (end 81 100.75) (width 0.2) (layer "F.Cu") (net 17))
 (segment (start 104 101.27) (end 119 100.75) (width 0.2) (layer "F.Cu") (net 17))
 (segment (start 98.73 102.54) (end 101.27 101.27) (width 0.2) (layer "F.Cu") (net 17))
 (segment (start 81 100.75) (end 96 102.54) (width 0.2) (layer "F.Cu") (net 17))
 (segment (start 119 100.75) (end 120.2 100.75) (width 0.2) (layer "F.Cu") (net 17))
 (segment (start 104 102.54) (end 119 101.25) (width 0.2) (layer "F.Cu") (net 18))
 (segment (start 119 101.25) (end 120.2 101.25) (width 0.2) (layer "F.Cu") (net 18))
 (segment (start 81 101.25) (end 96 103.81) (width 0.2) (layer "F.Cu") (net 18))
 (segment (start 79.8 101.25) (end 81 101.25) (width 0.2) (layer "F.Cu") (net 18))
 (segment (start 98.73 103.81) (end 101.27 102.54) (width 0.2) (layer "F.Cu") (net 18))
 (segment (start 96 103.81) (end 98.73 103.81) (width 0.2) (layer "F.Cu") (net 18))
 (segment (start 101.27 102.54) (end 104 102.54) (width 0.2) (layer "F.Cu") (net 18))
 (segment (start 98.73 105.08) (end 101.27 103.81) (width 0.2) (layer "F.Cu") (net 19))
 (segment (start 104 103.81) (end 119 101.75) (width 0.2) (layer "F.Cu") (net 19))
 (segment (start 79.8 101.75) (end 81 101.75) (width 0.2) (layer "F.Cu") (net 19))
 (segment (start 81 101.75) (end 96 105.08) (width 0.2) (layer "F.Cu") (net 19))
 (segment (start 119 101.75) (end 120.2 101.75) (width 0.2) (layer "F.Cu") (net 19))
 (segment (start 101.27 103.81) (end 104 103.81) (width 0.2) (layer "F.Cu") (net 19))
 (segment (start 96 105.08) (end 98.73 105.08) (width 0.2) (layer "F.Cu") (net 19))
 (segment (start 119 102.25) (end 120.2 102.25) (width 0.2) (layer "F.Cu") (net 20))
 (segment (start 104 105.08) (end 119 102.25) (width 0.2) (layer "F.Cu") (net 20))
 (segment (start 101.27 105.08) (end 104 105.08) (width 0.2) (layer "F.Cu") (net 20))
 (segment (start 98.73 106.35) (end 101.27 105.08) (width 0.2) (layer "F.Cu") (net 20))
 (segment (start 96 106.35) (end 98.73 106.35) (width 0.2) (layer "F.Cu") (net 20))
 (segment (start 81 102.25) (end 96 106.35) (width 0.2) (layer "F.Cu") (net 20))
 (segment (start 79.8 102.25) (end 81 102.25) (width 0.2) (layer "F.Cu") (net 20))
 (segment (start 96 107.62) (end 98.73 107.62) (width 0.2) (layer "F.Cu") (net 21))
 (segment (start 81 102.75) (end 96 107.62) (width 0.2) (layer "F.Cu") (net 21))
 (segment (start 104 106.35) (end 119 102.75) (width 0.2) (layer "F.Cu") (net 21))
 (segment (start 101.27 106.35) (end 104 106.35) (width 0.2) (layer "F.Cu") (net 21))
 (segment (start 119 102.75) (end 120.2 102.75) (width 0.2) (layer "F.Cu") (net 21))
 (segment (start 98.73 107.62) (end 101.27 106.35) (width 0.2) (layer "F.Cu") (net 21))
 (segment (start 79.8 102.75) (end 81 102.75) (width 0.2) (layer "F.Cu") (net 21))
 (segment (start 96 108.89) (end 98.73 108.89) (width 0.2) (layer "F.Cu") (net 22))
 (segment (start 101.27 107.62) (end 104 107.62) (width 0.2) (layer "F.Cu") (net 22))
 (segment (start 104 107.62) (end 119 103.25) (width 0.2) (layer "F.Cu") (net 22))
 (segment (start 81 103.25) (end 96 108.89) (width 0.2) (layer "F.Cu") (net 22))
 (segment (start 79.8 103.25) (end 81 103.25) (width 0.2) (layer "F.Cu") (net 22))
 (segment (start 119 103.25) (end 120.2 103.25) (width 0.2) (layer "F.Cu") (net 22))
 (segment (start 98.73 108.89) (end 101.27 107.62) (width 0.2) (layer "F.Cu") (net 22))
 (segment (start 81 103.75) (end 96 110.16) (width 0.2) (layer "F.Cu") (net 23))
 (segment (start 96 110.16) (end 98.73 110.16) (width 0.2) (layer "F.Cu") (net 23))
 (segment (start 98.73 110.16) (end 101.27 108.89) (width 0.2) (layer "F.Cu") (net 23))
 (segment (start 104 108.89) (end 119 103.75) (width 0.2) (layer "F.Cu") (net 23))
 (segment (start 101.27 108.89) (end 104 108.89) (width 0.2) (layer "F.Cu") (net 23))
 (segment (start 79.8 103.75) (end 81 103.75) (width 0.2) (layer "F.Cu") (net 23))
 (segment (start 119 103.75) (end 120.2 103.75) (width 0.2) (layer "F.Cu") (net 23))
 (segment (start 96 111.43) (end 98.73 111.43) (width 0.2) (layer "F.Cu") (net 24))
 (segment (start 119 104.25) (end 120.2 104.25) (width 0.2) (layer "F.Cu") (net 24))
 (segment (start 81 104.25) (end 96 111.43) (width 0.2) (layer "F.Cu") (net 24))
 (segment (start 104 110.16) (end 119 104.25) (width 0.2) (layer "F.Cu") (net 24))
 (segment (start 98.73 111.43) (end 101.27 110.16) (width 0.2) (layer "F.Cu") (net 24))
 (segment (start 101.27 110.16) (end 104 110.16) (width 0.2) (layer "F.Cu") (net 24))
 (segment (start 79.8 104.25) (end 81 104.25) (width 0.2) (layer "F.Cu") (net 24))
 (segment (start 98.73 112.7) (end 101.27 111.43) (width 0.2) (layer "F.Cu") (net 25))
 (segment (start 79.8 104.75) (end 81 104.75) (width 0.2) (layer "F.Cu") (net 25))
 (segment (start 101.27 111.43) (end 104 111.43) (width 0.2) (layer "F.Cu") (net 25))
 (segment (start 104 111.43) (end 119 104.75) (width 0.2) (layer "F.Cu") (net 25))
 (segment (start 96 112.7) (end 98.73 112.7) (width 0.2) (layer "F.Cu") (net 25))
 (segment (start 81 104.75) (end 96 112.7) (width 0.2) (layer "F.Cu") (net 25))
 (segment (start 119 104.75) (end 120.2 104.75) (width 0.2) (layer "F.Cu") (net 25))
 (segment (start 96 113.97) (end 98.73 113.97) (width 0.2) (layer "F.Cu") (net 26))
 (segment (start 98.73 113.97) (end 101.27 112.7) (width 0.2) (layer "F.Cu") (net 26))
 (segment (start 101.27 112.7) (end 104 112.7) (width 0.2) (layer "F.Cu") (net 26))
 (segment (start 119 105.25) (end 120.2 105.25) (width 0.2) (layer "F.Cu") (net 26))
 (segment (start 79.8 105.25) (end 81 105.25) (width 0.2) (layer "F.Cu") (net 26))
 (segment (start 104 112.7) (end 119 105.25) (width 0.2) (layer "F.Cu") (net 26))
 (segment (start 81 105.25) (end 96 113.97) (width 0.2) (layer "F.Cu") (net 26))
 (segment (start 98.73 115.24) (end 101.27 113.97) (width 0.2) (layer "F.Cu") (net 27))
 (segment (start 79.8 105.75) (end 81 105.75) (width 0.2) (layer "F.Cu") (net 27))
 (segment (start 104 113.97) (end 119 105.75) (width 0.2) (layer "F.Cu") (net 27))
 (segment (start 119 105.75) (end 120.2 105.75) (width 0.2) (layer "F.Cu") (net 27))
 (segment (start 81 105.75) (end 96 115.24) (width 0.2) (layer "F.Cu") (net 27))
 (segment (start 96 115.24) (end 98.73 115.24) (width 0.2) (layer "F.Cu") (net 27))
 (segment (start 101.27 113.97) (end 104 113.97) (width 0.2) (layer "F.Cu") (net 27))
 (segment (start 96 116.509999) (end 98.73 116.509999) (width 0.2) (layer "F.Cu") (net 28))
 (segment (start 101.27 115.24) (end 104 115.24) (width 0.2) (layer "F.Cu") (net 28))
 (segment (start 81 106.25) (end 96 116.509999) (width 0.2) (layer "F.Cu") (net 28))
 (segment (start 104 115.24) (end 119 106.25) (width 0.2) (layer "F.Cu") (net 28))
 (segment (start 98.73 116.509999) (end 101.27 115.24) (width 0.2) (layer "F.Cu") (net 28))
 (segment (start 79.8 106.25) (end 81 106.25) (width 0.2) (layer "F.Cu") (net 28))
 (segment (start 119 106.25) (end 120.2 106.25) (width 0.2) (layer "F.Cu") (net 28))
 (segment (start 101.27 116.51) (end 104 116.51) (width 0.2) (layer "F.Cu") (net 29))
 (segment (start 81 106.75) (end 96 117.78) (width 0.2) (layer "F.Cu") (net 29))
 (segment (start 79.8 106.75) (end 81 106.75) (width 0.2) (layer "F.Cu") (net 29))
 (segment (start 119 106.75) (end 120.2 106.75) (width 0.2) (layer "F.Cu") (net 29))
 (segment (start 98.73 117.78) (end 101.27 116.51) (width 0.2) (layer "F.Cu") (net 29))
 (segment (start 104 116.51) (end 119 106.75) (width 0.2) (layer "F.Cu") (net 29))
 (segment (start 96 117.78) (end 98.73 117.78) (width 0.2) (layer "F.Cu") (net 29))
 (segment (start 79.8 107.25) (end 81 107.25) (width 0.2) (layer "F.Cu") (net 30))
 (segment (start 96 119.05) (end 98.73 119.05) (width 0.2) (layer "F.Cu") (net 30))
 (segment (start 104 117.78) (end 119 107.25) (width 0.2) (layer "F.Cu") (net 30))
 (segment (start 98.73 119.05) (end 101.27 117.78) (width 0.2) (layer "F.Cu") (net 30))
 (segment (start 81 107.25) (end 96 119.05) (width 0.2) (layer "F.Cu") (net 30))
 (segment (start 101.27 117.78) (end 104 117.78) (width 0.2) (layer "F.Cu") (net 30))
 (segment (start 119 107.25) (end 120.2 107.25) (width 0.2) (layer "F.Cu") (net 30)))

